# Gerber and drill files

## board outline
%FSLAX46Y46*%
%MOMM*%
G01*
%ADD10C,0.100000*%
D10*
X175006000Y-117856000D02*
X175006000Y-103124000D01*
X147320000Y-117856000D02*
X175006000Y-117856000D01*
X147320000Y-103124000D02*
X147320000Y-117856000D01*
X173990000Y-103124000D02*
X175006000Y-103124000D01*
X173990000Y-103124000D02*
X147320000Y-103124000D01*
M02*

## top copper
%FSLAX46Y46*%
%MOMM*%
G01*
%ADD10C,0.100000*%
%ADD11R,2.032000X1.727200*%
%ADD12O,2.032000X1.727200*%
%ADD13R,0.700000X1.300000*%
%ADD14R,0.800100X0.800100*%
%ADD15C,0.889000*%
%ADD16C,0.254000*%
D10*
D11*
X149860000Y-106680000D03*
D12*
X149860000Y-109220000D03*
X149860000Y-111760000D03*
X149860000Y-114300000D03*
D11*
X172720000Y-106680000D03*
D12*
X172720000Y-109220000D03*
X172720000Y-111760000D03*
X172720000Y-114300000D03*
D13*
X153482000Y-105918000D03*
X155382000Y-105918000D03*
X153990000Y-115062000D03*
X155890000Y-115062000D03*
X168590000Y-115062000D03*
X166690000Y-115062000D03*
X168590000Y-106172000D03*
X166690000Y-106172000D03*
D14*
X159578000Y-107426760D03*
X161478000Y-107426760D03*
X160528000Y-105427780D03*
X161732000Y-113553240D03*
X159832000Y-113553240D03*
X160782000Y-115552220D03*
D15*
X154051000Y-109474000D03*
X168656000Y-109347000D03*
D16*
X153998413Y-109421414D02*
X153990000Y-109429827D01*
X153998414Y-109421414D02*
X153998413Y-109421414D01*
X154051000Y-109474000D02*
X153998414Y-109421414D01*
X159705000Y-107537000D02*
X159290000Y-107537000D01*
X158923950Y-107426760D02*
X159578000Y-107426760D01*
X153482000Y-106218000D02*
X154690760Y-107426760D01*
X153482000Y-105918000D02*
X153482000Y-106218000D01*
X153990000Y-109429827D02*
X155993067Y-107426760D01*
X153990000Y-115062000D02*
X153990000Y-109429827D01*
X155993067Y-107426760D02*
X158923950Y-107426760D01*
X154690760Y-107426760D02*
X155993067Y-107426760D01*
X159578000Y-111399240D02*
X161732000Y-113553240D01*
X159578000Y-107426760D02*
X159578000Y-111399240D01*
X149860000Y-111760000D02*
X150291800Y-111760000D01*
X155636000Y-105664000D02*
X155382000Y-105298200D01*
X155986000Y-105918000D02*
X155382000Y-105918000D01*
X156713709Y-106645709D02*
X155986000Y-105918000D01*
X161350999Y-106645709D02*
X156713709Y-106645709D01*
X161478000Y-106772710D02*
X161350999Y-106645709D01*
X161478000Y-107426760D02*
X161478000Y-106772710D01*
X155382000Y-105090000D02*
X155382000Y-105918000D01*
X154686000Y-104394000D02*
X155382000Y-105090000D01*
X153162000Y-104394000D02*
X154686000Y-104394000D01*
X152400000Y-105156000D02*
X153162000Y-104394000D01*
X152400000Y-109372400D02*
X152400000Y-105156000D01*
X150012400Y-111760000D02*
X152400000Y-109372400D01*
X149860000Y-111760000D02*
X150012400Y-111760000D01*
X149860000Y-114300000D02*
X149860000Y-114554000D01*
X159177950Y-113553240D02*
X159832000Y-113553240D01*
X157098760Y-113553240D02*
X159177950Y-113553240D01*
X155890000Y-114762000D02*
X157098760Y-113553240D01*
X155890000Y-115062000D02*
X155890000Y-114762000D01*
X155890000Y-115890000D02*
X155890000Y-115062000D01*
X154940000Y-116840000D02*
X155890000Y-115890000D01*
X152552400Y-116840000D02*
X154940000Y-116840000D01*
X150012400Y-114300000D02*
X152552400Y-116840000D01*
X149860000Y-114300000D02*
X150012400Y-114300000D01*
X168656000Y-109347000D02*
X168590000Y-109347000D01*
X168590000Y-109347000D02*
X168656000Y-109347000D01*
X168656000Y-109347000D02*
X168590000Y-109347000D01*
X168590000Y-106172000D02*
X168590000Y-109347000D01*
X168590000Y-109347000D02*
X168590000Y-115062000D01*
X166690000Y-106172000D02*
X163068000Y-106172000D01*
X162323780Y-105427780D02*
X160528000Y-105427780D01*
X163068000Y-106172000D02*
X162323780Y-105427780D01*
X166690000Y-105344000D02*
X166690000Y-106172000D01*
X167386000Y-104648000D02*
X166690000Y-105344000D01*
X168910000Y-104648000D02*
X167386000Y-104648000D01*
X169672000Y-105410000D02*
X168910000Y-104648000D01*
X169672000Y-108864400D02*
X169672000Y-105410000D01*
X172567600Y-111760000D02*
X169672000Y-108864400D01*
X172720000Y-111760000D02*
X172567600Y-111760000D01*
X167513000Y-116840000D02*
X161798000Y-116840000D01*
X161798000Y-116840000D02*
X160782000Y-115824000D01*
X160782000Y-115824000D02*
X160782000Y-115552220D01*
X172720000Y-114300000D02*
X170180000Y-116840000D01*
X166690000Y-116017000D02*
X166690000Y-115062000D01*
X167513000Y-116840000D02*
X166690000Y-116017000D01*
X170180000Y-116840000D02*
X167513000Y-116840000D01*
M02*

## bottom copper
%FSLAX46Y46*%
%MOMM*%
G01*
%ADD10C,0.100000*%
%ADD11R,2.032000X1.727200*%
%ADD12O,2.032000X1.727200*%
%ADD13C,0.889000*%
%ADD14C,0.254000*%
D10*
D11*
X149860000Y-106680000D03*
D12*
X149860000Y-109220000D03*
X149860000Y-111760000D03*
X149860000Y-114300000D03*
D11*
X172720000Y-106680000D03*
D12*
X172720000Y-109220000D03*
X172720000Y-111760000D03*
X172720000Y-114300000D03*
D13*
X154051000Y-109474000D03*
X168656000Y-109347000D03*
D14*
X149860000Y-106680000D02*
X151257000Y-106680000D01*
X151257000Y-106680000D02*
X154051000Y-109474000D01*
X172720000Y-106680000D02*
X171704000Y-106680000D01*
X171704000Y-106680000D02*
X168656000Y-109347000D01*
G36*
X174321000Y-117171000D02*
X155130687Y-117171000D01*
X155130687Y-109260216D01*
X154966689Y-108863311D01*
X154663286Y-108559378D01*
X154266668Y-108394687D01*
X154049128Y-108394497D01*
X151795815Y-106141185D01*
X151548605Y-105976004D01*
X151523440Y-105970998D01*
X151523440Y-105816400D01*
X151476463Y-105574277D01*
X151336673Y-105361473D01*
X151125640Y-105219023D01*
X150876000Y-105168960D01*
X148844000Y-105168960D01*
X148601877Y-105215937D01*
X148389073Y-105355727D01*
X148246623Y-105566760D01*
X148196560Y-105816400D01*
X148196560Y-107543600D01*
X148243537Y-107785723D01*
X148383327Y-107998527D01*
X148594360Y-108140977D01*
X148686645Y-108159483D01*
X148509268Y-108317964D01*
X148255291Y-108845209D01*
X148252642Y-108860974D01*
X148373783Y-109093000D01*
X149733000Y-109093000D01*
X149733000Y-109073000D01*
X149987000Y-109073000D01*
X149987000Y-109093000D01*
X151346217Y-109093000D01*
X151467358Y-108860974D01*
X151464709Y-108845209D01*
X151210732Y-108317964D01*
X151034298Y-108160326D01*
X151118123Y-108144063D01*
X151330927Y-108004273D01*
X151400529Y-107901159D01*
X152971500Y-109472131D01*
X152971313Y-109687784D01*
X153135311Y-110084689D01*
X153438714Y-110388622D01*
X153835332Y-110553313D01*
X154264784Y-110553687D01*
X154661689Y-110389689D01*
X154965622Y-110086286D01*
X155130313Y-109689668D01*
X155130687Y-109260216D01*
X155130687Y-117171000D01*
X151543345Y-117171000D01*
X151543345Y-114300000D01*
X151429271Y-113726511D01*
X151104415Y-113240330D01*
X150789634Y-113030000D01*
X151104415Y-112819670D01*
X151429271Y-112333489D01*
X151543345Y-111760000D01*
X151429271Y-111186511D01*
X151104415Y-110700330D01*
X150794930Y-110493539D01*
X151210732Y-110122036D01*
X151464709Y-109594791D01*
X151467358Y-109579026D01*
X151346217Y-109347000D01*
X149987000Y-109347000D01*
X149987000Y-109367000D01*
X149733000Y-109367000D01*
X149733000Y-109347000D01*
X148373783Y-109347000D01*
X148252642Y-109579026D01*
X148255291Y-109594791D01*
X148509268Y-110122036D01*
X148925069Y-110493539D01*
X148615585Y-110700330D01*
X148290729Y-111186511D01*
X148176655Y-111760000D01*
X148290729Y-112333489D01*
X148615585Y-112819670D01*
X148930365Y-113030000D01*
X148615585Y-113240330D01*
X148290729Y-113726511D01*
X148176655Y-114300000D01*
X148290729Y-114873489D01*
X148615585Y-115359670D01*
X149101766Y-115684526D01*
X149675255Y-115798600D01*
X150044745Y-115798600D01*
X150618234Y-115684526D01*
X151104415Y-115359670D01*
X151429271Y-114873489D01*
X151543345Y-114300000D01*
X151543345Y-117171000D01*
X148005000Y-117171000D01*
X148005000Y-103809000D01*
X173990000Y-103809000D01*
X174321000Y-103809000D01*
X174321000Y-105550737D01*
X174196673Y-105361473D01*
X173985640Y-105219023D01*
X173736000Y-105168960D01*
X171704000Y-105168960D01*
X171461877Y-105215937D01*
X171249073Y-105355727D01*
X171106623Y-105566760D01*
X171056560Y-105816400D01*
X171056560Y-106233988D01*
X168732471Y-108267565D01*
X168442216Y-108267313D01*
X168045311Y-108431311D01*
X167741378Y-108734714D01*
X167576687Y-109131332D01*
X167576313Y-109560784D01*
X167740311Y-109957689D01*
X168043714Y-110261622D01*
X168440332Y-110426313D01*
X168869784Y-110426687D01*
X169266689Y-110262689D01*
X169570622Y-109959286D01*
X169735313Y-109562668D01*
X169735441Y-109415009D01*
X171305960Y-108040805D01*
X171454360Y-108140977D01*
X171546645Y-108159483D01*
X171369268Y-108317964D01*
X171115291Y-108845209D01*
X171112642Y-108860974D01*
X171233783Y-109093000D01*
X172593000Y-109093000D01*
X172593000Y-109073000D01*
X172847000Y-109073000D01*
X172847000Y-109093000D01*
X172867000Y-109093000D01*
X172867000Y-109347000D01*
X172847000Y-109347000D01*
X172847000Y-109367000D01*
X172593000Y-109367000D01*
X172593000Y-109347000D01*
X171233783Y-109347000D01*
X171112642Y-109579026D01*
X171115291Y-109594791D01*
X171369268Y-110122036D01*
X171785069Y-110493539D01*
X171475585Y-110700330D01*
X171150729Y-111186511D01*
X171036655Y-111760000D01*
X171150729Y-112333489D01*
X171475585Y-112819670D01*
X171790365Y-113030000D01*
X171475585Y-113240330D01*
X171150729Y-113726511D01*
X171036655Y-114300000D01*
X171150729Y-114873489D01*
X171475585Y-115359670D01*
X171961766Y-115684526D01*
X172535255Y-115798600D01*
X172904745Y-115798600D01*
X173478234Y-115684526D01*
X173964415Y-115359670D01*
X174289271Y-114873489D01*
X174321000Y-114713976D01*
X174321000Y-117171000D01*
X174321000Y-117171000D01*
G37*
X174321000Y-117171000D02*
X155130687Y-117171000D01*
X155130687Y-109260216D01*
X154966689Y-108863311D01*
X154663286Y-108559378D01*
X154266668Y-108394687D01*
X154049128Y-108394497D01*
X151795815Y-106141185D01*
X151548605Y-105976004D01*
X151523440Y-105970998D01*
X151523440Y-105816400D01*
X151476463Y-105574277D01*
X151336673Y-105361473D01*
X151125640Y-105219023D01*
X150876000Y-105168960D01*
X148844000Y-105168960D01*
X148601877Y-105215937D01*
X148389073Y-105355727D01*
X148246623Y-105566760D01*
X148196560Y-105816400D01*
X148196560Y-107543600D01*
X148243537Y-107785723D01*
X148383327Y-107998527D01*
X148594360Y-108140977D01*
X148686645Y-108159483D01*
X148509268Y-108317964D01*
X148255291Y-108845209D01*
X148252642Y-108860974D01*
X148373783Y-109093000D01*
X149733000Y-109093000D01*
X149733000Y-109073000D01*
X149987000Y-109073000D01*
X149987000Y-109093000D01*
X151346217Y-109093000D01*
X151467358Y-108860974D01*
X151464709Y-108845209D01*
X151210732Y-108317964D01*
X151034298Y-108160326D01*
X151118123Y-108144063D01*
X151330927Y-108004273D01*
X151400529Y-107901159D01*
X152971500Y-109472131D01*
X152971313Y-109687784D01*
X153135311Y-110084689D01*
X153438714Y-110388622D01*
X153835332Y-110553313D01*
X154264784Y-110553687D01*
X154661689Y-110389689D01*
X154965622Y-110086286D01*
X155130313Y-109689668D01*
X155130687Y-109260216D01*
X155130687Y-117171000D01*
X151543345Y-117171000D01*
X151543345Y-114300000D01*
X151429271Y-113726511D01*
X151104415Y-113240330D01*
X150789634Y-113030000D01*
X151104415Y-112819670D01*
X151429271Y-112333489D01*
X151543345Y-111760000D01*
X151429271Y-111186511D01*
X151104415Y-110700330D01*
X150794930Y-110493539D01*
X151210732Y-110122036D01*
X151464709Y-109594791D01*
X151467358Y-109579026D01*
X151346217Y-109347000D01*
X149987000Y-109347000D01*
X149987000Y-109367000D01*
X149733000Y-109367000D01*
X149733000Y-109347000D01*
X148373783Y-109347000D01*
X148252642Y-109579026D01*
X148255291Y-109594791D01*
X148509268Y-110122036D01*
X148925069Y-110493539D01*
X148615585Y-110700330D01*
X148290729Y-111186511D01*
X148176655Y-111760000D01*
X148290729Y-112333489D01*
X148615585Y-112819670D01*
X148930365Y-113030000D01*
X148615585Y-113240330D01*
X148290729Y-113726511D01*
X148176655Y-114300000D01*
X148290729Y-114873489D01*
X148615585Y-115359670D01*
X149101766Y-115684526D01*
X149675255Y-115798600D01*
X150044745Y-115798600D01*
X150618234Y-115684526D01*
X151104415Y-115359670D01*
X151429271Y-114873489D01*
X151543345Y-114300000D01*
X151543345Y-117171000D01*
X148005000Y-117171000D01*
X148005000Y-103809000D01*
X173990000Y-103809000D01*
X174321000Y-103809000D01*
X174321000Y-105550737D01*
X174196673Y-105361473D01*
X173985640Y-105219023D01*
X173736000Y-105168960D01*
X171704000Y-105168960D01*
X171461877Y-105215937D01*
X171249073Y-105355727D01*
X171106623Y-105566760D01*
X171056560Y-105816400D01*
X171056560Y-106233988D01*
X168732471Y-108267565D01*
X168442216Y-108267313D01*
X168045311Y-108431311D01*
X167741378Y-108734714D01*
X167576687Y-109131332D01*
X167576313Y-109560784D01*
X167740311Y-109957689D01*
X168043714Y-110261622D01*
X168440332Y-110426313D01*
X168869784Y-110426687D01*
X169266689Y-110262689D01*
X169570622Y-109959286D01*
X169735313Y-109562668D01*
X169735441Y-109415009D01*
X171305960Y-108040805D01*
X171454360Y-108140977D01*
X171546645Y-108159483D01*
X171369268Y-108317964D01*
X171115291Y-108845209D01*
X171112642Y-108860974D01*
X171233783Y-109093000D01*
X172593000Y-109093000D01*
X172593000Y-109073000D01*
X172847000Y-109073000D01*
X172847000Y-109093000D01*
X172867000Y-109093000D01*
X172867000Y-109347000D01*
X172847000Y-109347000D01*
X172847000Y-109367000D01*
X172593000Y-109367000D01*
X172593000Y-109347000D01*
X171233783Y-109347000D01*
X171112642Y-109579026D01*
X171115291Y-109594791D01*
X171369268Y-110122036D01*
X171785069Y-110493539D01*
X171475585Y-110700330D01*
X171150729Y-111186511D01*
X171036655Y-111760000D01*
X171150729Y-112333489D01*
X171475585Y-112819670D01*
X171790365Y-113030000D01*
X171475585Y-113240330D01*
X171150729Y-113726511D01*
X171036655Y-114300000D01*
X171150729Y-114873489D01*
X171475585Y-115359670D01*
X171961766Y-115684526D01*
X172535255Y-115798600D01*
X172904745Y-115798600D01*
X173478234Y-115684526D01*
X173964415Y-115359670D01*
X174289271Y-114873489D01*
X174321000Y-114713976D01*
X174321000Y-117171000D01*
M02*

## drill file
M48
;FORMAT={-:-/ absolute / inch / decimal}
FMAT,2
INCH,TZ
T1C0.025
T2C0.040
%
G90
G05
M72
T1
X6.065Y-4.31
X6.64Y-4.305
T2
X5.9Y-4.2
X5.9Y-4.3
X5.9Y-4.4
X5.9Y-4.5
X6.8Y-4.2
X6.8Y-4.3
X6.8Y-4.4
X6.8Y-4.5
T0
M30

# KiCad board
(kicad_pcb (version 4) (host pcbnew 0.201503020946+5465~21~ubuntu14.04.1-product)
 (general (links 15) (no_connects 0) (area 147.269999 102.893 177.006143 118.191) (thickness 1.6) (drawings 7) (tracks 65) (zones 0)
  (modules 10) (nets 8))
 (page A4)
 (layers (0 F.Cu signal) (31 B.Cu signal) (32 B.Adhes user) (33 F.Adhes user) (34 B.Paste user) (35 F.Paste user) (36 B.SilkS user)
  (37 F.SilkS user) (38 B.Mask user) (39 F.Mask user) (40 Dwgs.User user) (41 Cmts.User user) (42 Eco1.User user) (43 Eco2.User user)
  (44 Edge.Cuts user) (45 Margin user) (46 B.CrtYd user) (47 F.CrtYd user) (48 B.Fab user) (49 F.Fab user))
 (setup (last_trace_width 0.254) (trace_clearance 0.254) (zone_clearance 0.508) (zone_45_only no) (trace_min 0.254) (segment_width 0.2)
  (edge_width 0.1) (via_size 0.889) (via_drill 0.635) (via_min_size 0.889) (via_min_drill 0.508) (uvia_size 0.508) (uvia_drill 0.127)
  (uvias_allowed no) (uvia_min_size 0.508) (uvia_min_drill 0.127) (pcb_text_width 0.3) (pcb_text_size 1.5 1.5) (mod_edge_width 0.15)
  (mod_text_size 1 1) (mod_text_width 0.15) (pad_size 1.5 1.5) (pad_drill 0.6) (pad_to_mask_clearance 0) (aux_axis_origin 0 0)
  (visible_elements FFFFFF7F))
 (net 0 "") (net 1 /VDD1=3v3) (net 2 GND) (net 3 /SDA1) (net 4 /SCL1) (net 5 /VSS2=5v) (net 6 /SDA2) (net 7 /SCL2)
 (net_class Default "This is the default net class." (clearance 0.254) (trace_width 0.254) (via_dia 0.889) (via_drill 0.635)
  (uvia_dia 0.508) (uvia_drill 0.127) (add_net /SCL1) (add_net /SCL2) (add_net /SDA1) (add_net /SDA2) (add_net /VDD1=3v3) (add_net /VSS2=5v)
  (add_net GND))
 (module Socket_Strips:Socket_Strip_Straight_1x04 (layer F.Cu) (at 149.86 106.68 270)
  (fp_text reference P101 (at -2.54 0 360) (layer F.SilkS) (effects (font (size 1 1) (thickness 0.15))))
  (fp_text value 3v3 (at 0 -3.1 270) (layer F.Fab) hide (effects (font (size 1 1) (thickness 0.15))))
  (pad 1 thru_hole rect (at 0 0 270) (size 1.7272 2.032) (drill 1.016) (layers *.Cu *.Mask F.SilkS) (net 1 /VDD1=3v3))
  (pad 2 thru_hole oval (at 2.54 0 270) (size 1.7272 2.032) (drill 1.016) (layers *.Cu *.Mask F.SilkS) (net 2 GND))
  (pad 3 thru_hole oval (at 5.08 0 270) (size 1.7272 2.032) (drill 1.016) (layers *.Cu *.Mask F.SilkS) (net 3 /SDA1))
  (pad 4 thru_hole oval (at 7.62 0 270) (size 1.7272 2.032) (drill 1.016) (layers *.Cu *.Mask F.SilkS) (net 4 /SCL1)))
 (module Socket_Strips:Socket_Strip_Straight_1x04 (layer F.Cu) (at 172.72 106.68 270)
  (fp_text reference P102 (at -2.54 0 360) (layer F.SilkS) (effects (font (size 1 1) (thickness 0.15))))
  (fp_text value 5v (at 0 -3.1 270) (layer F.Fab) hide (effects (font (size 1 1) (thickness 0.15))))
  (pad 1 thru_hole rect (at 0 0 270) (size 1.7272 2.032) (drill 1.016) (layers *.Cu *.Mask F.SilkS) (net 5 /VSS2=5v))
  (pad 2 thru_hole oval (at 2.54 0 270) (size 1.7272 2.032) (drill 1.016) (layers *.Cu *.Mask F.SilkS) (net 2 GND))
  (pad 3 thru_hole oval (at 5.08 0 270) (size 1.7272 2.032) (drill 1.016) (layers *.Cu *.Mask F.SilkS) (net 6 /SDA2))
  (pad 4 thru_hole oval (at 7.62 0 270) (size 1.7272 2.032) (drill 1.016) (layers *.Cu *.Mask F.SilkS) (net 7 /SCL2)))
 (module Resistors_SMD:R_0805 (layer F.Cu) (at 154.432 105.918)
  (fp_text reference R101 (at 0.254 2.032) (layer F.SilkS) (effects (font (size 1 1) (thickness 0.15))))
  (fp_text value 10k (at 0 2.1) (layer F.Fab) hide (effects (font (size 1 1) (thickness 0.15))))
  (pad 1 smd rect (at -0.95 0) (size 0.7 1.3) (layers F.Cu F.Paste F.Mask) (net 1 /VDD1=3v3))
  (pad 2 smd rect (at 0.95 0) (size 0.7 1.3) (layers F.Cu F.Paste F.Mask) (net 3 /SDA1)))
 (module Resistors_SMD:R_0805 (layer F.Cu) (at 154.94 115.062)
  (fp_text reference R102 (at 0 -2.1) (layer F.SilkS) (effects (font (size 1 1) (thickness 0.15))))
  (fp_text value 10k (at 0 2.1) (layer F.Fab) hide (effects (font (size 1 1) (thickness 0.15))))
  (pad 1 smd rect (at -0.95 0) (size 0.7 1.3) (layers F.Cu F.Paste F.Mask) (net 1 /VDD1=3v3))
  (pad 2 smd rect (at 0.95 0) (size 0.7 1.3) (layers F.Cu F.Paste F.Mask) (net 4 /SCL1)))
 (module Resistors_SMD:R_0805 (layer F.Cu) (at 167.64 115.062 180)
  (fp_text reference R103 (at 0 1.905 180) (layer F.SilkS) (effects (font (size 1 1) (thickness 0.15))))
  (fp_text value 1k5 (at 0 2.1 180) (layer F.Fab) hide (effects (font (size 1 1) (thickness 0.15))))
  (pad 1 smd rect (at -0.95 0 180) (size 0.7 1.3) (layers F.Cu F.Paste F.Mask) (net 5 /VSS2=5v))
  (pad 2 smd rect (at 0.95 0 180) (size 0.7 1.3) (layers F.Cu F.Paste F.Mask) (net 7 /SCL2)))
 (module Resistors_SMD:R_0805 (layer F.Cu) (at 167.64 106.172 180)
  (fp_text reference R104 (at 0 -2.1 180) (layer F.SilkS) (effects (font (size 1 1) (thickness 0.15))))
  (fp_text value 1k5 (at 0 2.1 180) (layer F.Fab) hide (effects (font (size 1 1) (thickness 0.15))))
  (pad 1 smd rect (at -0.95 0 180) (size 0.7 1.3) (layers F.Cu F.Paste F.Mask) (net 5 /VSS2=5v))
  (pad 2 smd rect (at 0.95 0 180) (size 0.7 1.3) (layers F.Cu F.Paste F.Mask) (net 6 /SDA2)))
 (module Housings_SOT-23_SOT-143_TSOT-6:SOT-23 (layer F.Cu) (at 160.528 106.426)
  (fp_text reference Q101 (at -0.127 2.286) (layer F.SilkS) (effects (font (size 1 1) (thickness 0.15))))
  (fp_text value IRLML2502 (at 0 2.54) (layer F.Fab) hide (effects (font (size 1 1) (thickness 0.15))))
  (pad 1 smd rect (at -0.95 1.00076) (size 0.8001 0.8001) (layers F.Cu F.Paste F.Mask) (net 1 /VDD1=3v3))
  (pad 2 smd rect (at 0.95 1.00076) (size 0.8001 0.8001) (layers F.Cu F.Paste F.Mask) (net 3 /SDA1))
  (pad 3 smd rect (at 0 -0.99822) (size 0.8001 0.8001) (layers F.Cu F.Paste F.Mask) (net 6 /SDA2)))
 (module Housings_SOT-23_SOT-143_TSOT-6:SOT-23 (layer F.Cu) (at 160.782 114.554 180)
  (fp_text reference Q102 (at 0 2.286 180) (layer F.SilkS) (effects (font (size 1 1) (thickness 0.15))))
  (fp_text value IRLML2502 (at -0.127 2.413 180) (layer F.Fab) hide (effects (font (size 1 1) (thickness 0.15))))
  (pad 1 smd rect (at -0.95 1.00076 180) (size 0.8001 0.8001) (layers F.Cu F.Paste F.Mask) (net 1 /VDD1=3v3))
  (pad 2 smd rect (at 0.95 1.00076 180) (size 0.8001 0.8001) (layers F.Cu F.Paste F.Mask) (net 4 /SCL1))
  (pad 3 smd rect (at 0 -0.99822 180) (size 0.8001 0.8001) (layers F.Cu F.Paste F.Mask) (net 7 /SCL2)))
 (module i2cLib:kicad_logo (layer F.Cu) (at 164.338 110.998 90)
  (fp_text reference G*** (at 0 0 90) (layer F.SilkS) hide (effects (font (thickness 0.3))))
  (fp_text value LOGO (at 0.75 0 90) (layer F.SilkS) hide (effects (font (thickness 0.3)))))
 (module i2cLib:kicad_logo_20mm (layer B.Cu) (at 161.29 113.792 180)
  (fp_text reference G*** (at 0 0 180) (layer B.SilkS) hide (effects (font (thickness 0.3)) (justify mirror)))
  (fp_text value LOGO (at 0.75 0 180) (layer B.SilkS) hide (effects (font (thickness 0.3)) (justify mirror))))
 (gr_line (start 175.006 117.856) (end 175.006 103.124) (angle 90) (layer Edge.Cuts) (width 0.1))
 (gr_line (start 147.32 117.856) (end 175.006 117.856) (angle 90) (layer Edge.Cuts) (width 0.1))
 (gr_line (start 147.32 103.124) (end 147.32 117.856) (angle 90) (layer Edge.Cuts) (width 0.1))
 (gr_line (start 173.99 103.124) (end 175.006 103.124) (angle 90) (layer Edge.Cuts) (width 0.1))
 (gr_line (start 173.99 103.124) (end 147.32 103.124) (angle 90) (layer Edge.Cuts) (width 0.1))
 (segment (start 149.86 106.68) (end 151.257 106.68) (width 0.254) (layer B.Cu) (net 1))
 (segment (start 153.998413 109.421414) (end 153.99 109.429827) (width 0.254) (layer F.Cu) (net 1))
 (segment (start 153.998414 109.421414) (end 153.998413 109.421414) (width 0.254) (layer F.Cu) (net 1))
 (segment (start 154.051 109.474) (end 153.998414 109.421414) (width 0.254) (layer F.Cu) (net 1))
 (via (at 154.051 109.474) (size 0.889) (layers F.Cu B.Cu) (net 1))
 (segment (start 151.257 106.68) (end 154.051 109.474) (width 0.254) (layer B.Cu) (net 1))
 (segment (start 159.705 107.537) (end 159.29 107.537) (width 0.254) (layer F.Cu) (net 1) (status 30))
 (segment (start 158.92395 107.42676) (end 159.578 107.42676) (width 0.254) (layer F.Cu) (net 1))
 (segment (start 153.482 106.218) (end 154.69076 107.42676) (width 0.254) (layer F.Cu) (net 1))
 (segment (start 153.482 105.918) (end 153.482 106.218) (width 0.254) (layer F.Cu) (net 1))
 (segment (start 153.99 109.429827) (end 155.993067 107.42676) (width 0.254) (layer F.Cu) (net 1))
 (segment (start 153.99 115.062) (end 153.99 109.429827) (width 0.254) (layer F.Cu) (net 1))
 (segment (start 155.993067 107.42676) (end 158.92395 107.42676) (width 0.254) (layer F.Cu) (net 1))
 (segment (start 154.69076 107.42676) (end 155.993067 107.42676) (width 0.254) (layer F.Cu) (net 1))
 (segment (start 159.578 111.39924) (end 161.732 113.55324) (width 0.254) (layer F.Cu) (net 1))
 (segment (start 159.578 107.42676) (end 159.578 111.39924) (width 0.254) (layer F.Cu) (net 1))
 (segment (start 149.86 111.76) (end 150.2918 111.76) (width 0.254) (layer F.Cu) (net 3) (status 30))
 (segment (start 155.636 105.664) (end 155.382 105.2982) (width 0.254) (layer F.Cu) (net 3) (status 30))
 (segment (start 155.986 105.918) (end 155.382 105.918) (width 0.254) (layer F.Cu) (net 3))
 (segment (start 156.713709 106.645709) (end 155.986 105.918) (width 0.254) (layer F.Cu) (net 3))
 (segment (start 161.350999 106.645709) (end 156.713709 106.645709) (width 0.254) (layer F.Cu) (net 3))
 (segment (start 161.478 106.77271) (end 161.350999 106.645709) (width 0.254) (layer F.Cu) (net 3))
 (segment (start 161.478 107.42676) (end 161.478 106.77271) (width 0.254) (layer F.Cu) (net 3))
 (segment (start 155.382 105.09) (end 155.382 105.918) (width 0.254) (layer F.Cu) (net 3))
 (segment (start 154.686 104.394) (end 155.382 105.09) (width 0.254) (layer F.Cu) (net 3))
 (segment (start 153.162 104.394) (end 154.686 104.394) (width 0.254) (layer F.Cu) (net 3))
 (segment (start 152.4 105.156) (end 153.162 104.394) (width 0.254) (layer F.Cu) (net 3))
 (segment (start 152.4 109.3724) (end 152.4 105.156) (width 0.254) (layer F.Cu) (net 3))
 (segment (start 150.0124 111.76) (end 152.4 109.3724) (width 0.254) (layer F.Cu) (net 3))
 (segment (start 149.86 111.76) (end 150.0124 111.76) (width 0.254) (layer F.Cu) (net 3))
 (segment (start 149.86 114.3) (end 149.86 114.554) (width 0.254) (layer F.Cu) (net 4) (status 30))
 (segment (start 159.17795 113.55324) (end 159.832 113.55324) (width 0.254) (layer F.Cu) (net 4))
 (segment (start 157.09876 113.55324) (end 159.17795 113.55324) (width 0.254) (layer F.Cu) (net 4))
 (segment (start 155.89 114.762) (end 157.09876 113.55324) (width 0.254) (layer F.Cu) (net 4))
 (segment (start 155.89 115.062) (end 155.89 114.762) (width 0.254) (layer F.Cu) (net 4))
 (segment (start 155.89 115.89) (end 155.89 115.062) (width 0.254) (layer F.Cu) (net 4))
 (segment (start 154.94 116.84) (end 155.89 115.89) (width 0.254) (layer F.Cu) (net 4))
 (segment (start 152.5524 116.84) (end 154.94 116.84) (width 0.254) (layer F.Cu) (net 4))
 (segment (start 150.0124 114.3) (end 152.5524 116.84) (width 0.254) (layer F.Cu) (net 4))
 (segment (start 149.86 114.3) (end 150.0124 114.3) (width 0.254) (layer F.Cu) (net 4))
 (segment (start 172.72 106.68) (end 171.704 106.68) (width 0.254) (layer B.Cu) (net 5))
 (segment (start 171.704 106.68) (end 168.656 109.347) (width 0.254) (layer B.Cu) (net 5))
 (via (at 168.656 109.347) (size 0.889) (layers F.Cu B.Cu) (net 5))
 (segment (start 168.656 109.347) (end 168.59 109.347) (width 0.254) (layer F.Cu) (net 5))
 (segment (start 168.59 109.347) (end 168.656 109.347) (width 0.254) (layer F.Cu) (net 5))
 (segment (start 168.656 109.347) (end 168.59 109.347) (width 0.254) (layer F.Cu) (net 5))
 (segment (start 168.59 106.172) (end 168.59 109.347) (width 0.254) (layer F.Cu) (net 5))
 (segment (start 168.59 109.347) (end 168.59 115.062) (width 0.254) (layer F.Cu) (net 5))
 (segment (start 166.69 106.172) (end 163.068 106.172) (width 0.254) (layer F.Cu) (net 6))
 (segment (start 162.32378 105.42778) (end 160.528 105.42778) (width 0.254) (layer F.Cu) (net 6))
 (segment (start 163.068 106.172) (end 162.32378 105.42778) (width 0.254) (layer F.Cu) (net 6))
 (segment (start 166.69 105.344) (end 166.69 106.172) (width 0.254) (layer F.Cu) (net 6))
 (segment (start 167.386 104.648) (end 166.69 105.344) (width 0.254) (layer F.Cu) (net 6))
 (segment (start 168.91 104.648) (end 167.386 104.648) (width 0.254) (layer F.Cu) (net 6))
 (segment (start 169.672 105.41) (end 168.91 104.648) (width 0.254) (layer F.Cu) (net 6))
 (segment (start 169.672 108.8644) (end 169.672 105.41) (width 0.254) (layer F.Cu) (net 6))
 (segment (start 172.5676 111.76) (end 169.672 108.8644) (width 0.254) (layer F.Cu) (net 6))
 (segment (start 172.72 111.76) (end 172.5676 111.76) (width 0.254) (layer F.Cu) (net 6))
 (segment (start 167.513 116.84) (end 161.798 116.84) (width 0.254) (layer F.Cu) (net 7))
 (segment (start 161.798 116.84) (end 160.782 115.824) (width 0.254) (layer F.Cu) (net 7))
 (segment (start 160.782 115.824) (end 160.782 115.55222) (width 0.254) (layer F.Cu) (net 7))
 (segment (start 172.72 114.3) (end 170.18 116.84) (width 0.254) (layer F.Cu) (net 7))
 (segment (start 166.69 116.017) (end 166.69 115.062) (width 0.254) (layer F.Cu) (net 7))
 (segment (start 167.513 116.84) (end 166.69 116.017) (width 0.254) (layer F.Cu) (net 7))
 (segment (start 170.18 116.84) (end 167.513 116.84) (width 0.254) (layer F.Cu) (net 7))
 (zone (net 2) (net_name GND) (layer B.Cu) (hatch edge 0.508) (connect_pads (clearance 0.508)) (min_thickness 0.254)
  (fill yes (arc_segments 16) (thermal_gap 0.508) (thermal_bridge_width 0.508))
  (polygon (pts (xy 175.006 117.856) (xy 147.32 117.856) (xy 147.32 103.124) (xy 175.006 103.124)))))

